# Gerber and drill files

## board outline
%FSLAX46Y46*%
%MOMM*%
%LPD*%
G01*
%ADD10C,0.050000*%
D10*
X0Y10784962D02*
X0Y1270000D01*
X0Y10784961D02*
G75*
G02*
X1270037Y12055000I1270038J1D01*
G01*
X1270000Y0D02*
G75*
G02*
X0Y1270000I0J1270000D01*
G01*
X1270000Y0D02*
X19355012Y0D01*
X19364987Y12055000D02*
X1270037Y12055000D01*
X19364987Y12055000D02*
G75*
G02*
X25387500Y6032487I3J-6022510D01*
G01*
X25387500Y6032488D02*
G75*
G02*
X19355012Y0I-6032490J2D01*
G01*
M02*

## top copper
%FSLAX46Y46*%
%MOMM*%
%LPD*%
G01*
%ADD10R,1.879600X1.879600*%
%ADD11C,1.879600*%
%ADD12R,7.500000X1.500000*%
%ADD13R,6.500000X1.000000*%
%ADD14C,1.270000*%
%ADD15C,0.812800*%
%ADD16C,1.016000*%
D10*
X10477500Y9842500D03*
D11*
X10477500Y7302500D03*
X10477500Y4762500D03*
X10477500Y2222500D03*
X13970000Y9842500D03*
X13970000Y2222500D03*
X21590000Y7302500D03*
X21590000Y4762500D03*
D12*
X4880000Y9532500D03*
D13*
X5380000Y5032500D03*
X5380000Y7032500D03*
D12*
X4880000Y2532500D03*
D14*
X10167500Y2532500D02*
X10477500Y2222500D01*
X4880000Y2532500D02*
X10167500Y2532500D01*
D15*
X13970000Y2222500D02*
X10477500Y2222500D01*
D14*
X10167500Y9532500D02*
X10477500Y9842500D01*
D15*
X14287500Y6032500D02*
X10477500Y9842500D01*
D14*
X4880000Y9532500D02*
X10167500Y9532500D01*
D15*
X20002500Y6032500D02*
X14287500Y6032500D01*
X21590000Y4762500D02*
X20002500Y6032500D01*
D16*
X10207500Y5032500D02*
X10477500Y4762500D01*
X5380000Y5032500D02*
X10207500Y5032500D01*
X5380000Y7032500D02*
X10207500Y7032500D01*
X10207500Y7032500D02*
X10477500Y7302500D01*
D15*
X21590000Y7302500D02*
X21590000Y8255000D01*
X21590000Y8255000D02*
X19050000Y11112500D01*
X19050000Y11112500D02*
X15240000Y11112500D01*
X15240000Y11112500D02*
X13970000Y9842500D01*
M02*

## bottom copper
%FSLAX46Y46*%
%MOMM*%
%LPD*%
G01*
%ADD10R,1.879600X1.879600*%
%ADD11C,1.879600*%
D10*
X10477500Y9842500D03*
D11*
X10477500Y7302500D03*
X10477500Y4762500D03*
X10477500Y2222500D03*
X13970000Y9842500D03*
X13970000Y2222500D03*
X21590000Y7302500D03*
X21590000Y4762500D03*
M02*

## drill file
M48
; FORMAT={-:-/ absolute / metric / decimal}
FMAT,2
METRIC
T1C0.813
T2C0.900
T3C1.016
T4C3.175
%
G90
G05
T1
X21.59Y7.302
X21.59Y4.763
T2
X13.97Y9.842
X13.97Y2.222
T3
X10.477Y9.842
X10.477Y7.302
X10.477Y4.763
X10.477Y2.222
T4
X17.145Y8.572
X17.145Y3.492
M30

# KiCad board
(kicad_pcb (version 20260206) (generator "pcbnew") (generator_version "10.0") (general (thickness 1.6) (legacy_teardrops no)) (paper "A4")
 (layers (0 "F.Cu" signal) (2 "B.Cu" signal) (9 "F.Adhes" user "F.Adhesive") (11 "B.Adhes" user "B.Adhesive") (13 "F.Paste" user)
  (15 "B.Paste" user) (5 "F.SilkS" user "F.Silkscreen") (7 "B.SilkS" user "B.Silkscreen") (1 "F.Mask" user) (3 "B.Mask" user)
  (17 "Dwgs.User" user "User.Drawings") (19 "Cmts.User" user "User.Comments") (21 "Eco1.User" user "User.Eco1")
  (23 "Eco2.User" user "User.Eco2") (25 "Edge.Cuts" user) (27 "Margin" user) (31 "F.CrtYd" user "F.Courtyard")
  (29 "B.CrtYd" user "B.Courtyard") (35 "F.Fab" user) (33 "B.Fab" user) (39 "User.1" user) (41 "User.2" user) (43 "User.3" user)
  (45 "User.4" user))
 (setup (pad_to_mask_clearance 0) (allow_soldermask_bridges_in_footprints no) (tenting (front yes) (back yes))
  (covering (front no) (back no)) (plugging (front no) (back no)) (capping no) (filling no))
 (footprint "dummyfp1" (layer "F.Cu") (at 17.145 -3.4925)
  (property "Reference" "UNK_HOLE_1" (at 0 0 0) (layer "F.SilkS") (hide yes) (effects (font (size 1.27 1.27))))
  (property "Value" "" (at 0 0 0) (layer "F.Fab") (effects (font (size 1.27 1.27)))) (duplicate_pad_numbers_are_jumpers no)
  (pad "" np_thru_hole circle (at 0 0) (size 3.175 3.175) (drill 3.175) (layers "*.Cu" "*.Mask")))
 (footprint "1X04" (layer "F.Cu") (at 10.4775 -9.8425 -90)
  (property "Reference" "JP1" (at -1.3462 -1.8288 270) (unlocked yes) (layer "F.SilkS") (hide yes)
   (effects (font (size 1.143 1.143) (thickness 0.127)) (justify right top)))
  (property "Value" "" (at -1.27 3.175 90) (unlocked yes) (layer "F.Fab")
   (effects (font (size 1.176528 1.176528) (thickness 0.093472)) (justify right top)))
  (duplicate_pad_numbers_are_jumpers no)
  (pad "1" thru_hole rect (at 0 0) (size 1.8796 1.8796) (drill 1.016) (layers "*.Cu" "*.Mask") (remove_unused_layers no) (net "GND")
   (solder_mask_margin 0.0762) (thermal_bridge_angle 0))
  (pad "2" thru_hole circle (at 2.54 0) (size 1.8796 1.8796) (drill 1.016) (layers "*.Cu" "*.Mask") (remove_unused_layers no) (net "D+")
   (solder_mask_margin 0.0762) (thermal_bridge_angle 0))
  (pad "3" thru_hole circle (at 5.08 0) (size 1.8796 1.8796) (drill 1.016) (layers "*.Cu" "*.Mask") (remove_unused_layers no) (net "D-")
   (solder_mask_margin 0.0762) (thermal_bridge_angle 0))
  (pad "4" thru_hole circle (at 7.62 0) (size 1.8796 1.8796) (drill 1.016) (layers "*.Cu" "*.Mask") (remove_unused_layers no) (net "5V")
   (solder_mask_margin 0.0762) (thermal_bridge_angle 0)))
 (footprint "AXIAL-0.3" (layer "F.Cu") (at 13.97 -6.0325 -90)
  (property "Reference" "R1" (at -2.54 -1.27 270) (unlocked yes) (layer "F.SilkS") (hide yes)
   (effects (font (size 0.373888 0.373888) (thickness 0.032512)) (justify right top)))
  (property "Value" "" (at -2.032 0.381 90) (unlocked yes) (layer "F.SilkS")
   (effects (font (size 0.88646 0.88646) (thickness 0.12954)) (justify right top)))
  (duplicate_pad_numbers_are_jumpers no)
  (pad "P$1" thru_hole circle (at -3.81 0 270) (size 1.8796 1.8796) (drill 0.9) (layers "*.Cu" "*.Mask") (remove_unused_layers no)
   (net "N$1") (solder_mask_margin 0.0762) (thermal_bridge_angle 0))
  (pad "P$2" thru_hole circle (at 3.81 0 270) (size 1.8796 1.8796) (drill 0.9) (layers "*.Cu" "*.Mask") (remove_unused_layers no) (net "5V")
   (solder_mask_margin 0.0762) (thermal_bridge_angle 0)))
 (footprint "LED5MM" (layer "F.Cu") (at 21.59 -6.0325 -90)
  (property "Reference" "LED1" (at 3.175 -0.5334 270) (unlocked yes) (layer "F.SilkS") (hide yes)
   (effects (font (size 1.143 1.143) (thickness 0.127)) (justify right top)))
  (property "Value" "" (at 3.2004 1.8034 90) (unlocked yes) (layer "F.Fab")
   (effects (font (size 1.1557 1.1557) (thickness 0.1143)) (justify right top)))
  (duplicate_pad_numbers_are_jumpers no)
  (pad "A" thru_hole circle (at -1.27 0 270) (size 1.8796 1.8796) (drill 0.8128) (layers "*.Cu" "*.Mask") (remove_unused_layers no)
   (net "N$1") (solder_mask_margin 0.0762) (thermal_bridge_angle 0))
  (pad "K" thru_hole circle (at 1.27 0 270) (size 1.8796 1.8796) (drill 0.8128) (layers "*.Cu" "*.Mask") (remove_unused_layers no)
   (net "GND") (solder_mask_margin 0.0762) (thermal_bridge_angle 0)))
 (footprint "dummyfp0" (layer "F.Cu") (at 17.145 -8.5725)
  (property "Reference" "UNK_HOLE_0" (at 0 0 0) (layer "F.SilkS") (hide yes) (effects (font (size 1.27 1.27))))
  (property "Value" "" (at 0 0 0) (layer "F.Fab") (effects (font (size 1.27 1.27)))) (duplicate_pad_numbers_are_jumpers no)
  (pad "" np_thru_hole circle (at 0 0) (size 3.175 3.175) (drill 3.175) (layers "*.Cu" "*.Mask")))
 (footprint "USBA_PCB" (layer "F.Cu") (at 5.08 -6.0325)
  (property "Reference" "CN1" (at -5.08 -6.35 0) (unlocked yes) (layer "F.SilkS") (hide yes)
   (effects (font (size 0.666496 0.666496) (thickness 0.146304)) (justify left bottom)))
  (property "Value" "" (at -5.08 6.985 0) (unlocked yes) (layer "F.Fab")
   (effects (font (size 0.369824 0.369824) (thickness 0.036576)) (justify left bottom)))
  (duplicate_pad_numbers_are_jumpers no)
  (pad "GND" smd rect (at -0.2 -3.5) (size 7.5 1.5) (layers "F.Cu" "F.Mask" "F.Paste") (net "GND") (solder_mask_margin 0.0762)
   (solder_paste_margin 0) (thermal_bridge_angle 0))
  (pad "USB_NEG" smd rect (at 0.3 1) (size 6.5 1) (layers "F.Cu" "F.Mask" "F.Paste") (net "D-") (solder_mask_margin 0.0762)
   (solder_paste_margin 0) (thermal_bridge_angle 0))
  (pad "USB_PLUS" smd rect (at 0.3 -1) (size 6.5 1) (layers "F.Cu" "F.Mask" "F.Paste") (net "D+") (solder_mask_margin 0.0762)
   (solder_paste_margin 0) (thermal_bridge_angle 0))
  (pad "VCC" smd rect (at -0.2 3.5) (size 7.5 1.5) (layers "F.Cu" "F.Mask" "F.Paste") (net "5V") (solder_mask_margin 0.0762)
   (solder_paste_margin 0) (thermal_bridge_angle 0)))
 (gr_line (start 0 -10.784962) (end 0 -1.27) (stroke (width 0.05) (type solid)) (layer "Edge.Cuts"))
 (gr_arc (start 0 -10.784961) (mid 0.371985 -11.683014) (end 1.270037 -12.055) (stroke (width 0.05) (type solid)) (layer "Edge.Cuts"))
 (gr_arc (start 1.27 0) (mid 0.371974 -0.371974) (end 0 -1.27) (stroke (width 0.05) (type solid)) (layer "Edge.Cuts"))
 (gr_line (start 1.27 0) (end 19.355012 0) (stroke (width 0.05) (type solid)) (layer "Edge.Cuts"))
 (gr_line (start 19.364987 -12.055) (end 1.270037 -12.055) (stroke (width 0.05) (type solid)) (layer "Edge.Cuts"))
 (gr_arc (start 19.364987 -12.055) (mid 23.623547 -10.291047) (end 25.3875 -6.032487) (stroke (width 0.05) (type solid)) (layer "Edge.Cuts"))
 (gr_arc (start 25.3875 -6.032488) (mid 23.620625 -1.766875) (end 19.355012 0) (stroke (width 0.05) (type solid)) (layer "Edge.Cuts"))
 (segment (start 10.1675 -2.5325) (end 10.4775 -2.2225) (width 1.27) (layer "F.Cu") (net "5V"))
 (segment (start 4.88 -2.5325) (end 10.1675 -2.5325) (width 1.27) (layer "F.Cu") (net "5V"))
 (segment (start 13.97 -2.2225) (end 10.4775 -2.2225) (width 0.8128) (layer "F.Cu") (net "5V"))
 (segment (start 10.1675 -9.5325) (end 10.4775 -9.8425) (width 1.27) (layer "F.Cu") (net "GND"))
 (segment (start 14.2875 -6.0325) (end 10.4775 -9.8425) (width 0.8128) (layer "F.Cu") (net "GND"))
 (segment (start 4.88 -9.5325) (end 10.1675 -9.5325) (width 1.27) (layer "F.Cu") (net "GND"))
 (segment (start 20.0025 -6.0325) (end 14.2875 -6.0325) (width 0.8128) (layer "F.Cu") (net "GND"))
 (segment (start 21.59 -4.7625) (end 20.0025 -6.0325) (width 0.8128) (layer "F.Cu") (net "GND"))
 (segment (start 10.2075 -5.0325) (end 10.4775 -4.7625) (width 1.016) (layer "F.Cu") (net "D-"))
 (segment (start 5.38 -5.0325) (end 10.2075 -5.0325) (width 1.016) (layer "F.Cu") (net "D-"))
 (segment (start 5.38 -7.0325) (end 10.2075 -7.0325) (width 1.016) (layer "F.Cu") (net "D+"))
 (segment (start 10.2075 -7.0325) (end 10.4775 -7.3025) (width 1.016) (layer "F.Cu") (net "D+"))
 (segment (start 21.59 -7.3025) (end 21.59 -8.255) (width 0.8128) (layer "F.Cu") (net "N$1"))
 (segment (start 21.59 -8.255) (end 19.05 -11.1125) (width 0.8128) (layer "F.Cu") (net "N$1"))
 (segment (start 19.05 -11.1125) (end 15.24 -11.1125) (width 0.8128) (layer "F.Cu") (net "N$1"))
 (segment (start 15.24 -11.1125) (end 13.97 -9.8425) (width 0.8128) (layer "F.Cu") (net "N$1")))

